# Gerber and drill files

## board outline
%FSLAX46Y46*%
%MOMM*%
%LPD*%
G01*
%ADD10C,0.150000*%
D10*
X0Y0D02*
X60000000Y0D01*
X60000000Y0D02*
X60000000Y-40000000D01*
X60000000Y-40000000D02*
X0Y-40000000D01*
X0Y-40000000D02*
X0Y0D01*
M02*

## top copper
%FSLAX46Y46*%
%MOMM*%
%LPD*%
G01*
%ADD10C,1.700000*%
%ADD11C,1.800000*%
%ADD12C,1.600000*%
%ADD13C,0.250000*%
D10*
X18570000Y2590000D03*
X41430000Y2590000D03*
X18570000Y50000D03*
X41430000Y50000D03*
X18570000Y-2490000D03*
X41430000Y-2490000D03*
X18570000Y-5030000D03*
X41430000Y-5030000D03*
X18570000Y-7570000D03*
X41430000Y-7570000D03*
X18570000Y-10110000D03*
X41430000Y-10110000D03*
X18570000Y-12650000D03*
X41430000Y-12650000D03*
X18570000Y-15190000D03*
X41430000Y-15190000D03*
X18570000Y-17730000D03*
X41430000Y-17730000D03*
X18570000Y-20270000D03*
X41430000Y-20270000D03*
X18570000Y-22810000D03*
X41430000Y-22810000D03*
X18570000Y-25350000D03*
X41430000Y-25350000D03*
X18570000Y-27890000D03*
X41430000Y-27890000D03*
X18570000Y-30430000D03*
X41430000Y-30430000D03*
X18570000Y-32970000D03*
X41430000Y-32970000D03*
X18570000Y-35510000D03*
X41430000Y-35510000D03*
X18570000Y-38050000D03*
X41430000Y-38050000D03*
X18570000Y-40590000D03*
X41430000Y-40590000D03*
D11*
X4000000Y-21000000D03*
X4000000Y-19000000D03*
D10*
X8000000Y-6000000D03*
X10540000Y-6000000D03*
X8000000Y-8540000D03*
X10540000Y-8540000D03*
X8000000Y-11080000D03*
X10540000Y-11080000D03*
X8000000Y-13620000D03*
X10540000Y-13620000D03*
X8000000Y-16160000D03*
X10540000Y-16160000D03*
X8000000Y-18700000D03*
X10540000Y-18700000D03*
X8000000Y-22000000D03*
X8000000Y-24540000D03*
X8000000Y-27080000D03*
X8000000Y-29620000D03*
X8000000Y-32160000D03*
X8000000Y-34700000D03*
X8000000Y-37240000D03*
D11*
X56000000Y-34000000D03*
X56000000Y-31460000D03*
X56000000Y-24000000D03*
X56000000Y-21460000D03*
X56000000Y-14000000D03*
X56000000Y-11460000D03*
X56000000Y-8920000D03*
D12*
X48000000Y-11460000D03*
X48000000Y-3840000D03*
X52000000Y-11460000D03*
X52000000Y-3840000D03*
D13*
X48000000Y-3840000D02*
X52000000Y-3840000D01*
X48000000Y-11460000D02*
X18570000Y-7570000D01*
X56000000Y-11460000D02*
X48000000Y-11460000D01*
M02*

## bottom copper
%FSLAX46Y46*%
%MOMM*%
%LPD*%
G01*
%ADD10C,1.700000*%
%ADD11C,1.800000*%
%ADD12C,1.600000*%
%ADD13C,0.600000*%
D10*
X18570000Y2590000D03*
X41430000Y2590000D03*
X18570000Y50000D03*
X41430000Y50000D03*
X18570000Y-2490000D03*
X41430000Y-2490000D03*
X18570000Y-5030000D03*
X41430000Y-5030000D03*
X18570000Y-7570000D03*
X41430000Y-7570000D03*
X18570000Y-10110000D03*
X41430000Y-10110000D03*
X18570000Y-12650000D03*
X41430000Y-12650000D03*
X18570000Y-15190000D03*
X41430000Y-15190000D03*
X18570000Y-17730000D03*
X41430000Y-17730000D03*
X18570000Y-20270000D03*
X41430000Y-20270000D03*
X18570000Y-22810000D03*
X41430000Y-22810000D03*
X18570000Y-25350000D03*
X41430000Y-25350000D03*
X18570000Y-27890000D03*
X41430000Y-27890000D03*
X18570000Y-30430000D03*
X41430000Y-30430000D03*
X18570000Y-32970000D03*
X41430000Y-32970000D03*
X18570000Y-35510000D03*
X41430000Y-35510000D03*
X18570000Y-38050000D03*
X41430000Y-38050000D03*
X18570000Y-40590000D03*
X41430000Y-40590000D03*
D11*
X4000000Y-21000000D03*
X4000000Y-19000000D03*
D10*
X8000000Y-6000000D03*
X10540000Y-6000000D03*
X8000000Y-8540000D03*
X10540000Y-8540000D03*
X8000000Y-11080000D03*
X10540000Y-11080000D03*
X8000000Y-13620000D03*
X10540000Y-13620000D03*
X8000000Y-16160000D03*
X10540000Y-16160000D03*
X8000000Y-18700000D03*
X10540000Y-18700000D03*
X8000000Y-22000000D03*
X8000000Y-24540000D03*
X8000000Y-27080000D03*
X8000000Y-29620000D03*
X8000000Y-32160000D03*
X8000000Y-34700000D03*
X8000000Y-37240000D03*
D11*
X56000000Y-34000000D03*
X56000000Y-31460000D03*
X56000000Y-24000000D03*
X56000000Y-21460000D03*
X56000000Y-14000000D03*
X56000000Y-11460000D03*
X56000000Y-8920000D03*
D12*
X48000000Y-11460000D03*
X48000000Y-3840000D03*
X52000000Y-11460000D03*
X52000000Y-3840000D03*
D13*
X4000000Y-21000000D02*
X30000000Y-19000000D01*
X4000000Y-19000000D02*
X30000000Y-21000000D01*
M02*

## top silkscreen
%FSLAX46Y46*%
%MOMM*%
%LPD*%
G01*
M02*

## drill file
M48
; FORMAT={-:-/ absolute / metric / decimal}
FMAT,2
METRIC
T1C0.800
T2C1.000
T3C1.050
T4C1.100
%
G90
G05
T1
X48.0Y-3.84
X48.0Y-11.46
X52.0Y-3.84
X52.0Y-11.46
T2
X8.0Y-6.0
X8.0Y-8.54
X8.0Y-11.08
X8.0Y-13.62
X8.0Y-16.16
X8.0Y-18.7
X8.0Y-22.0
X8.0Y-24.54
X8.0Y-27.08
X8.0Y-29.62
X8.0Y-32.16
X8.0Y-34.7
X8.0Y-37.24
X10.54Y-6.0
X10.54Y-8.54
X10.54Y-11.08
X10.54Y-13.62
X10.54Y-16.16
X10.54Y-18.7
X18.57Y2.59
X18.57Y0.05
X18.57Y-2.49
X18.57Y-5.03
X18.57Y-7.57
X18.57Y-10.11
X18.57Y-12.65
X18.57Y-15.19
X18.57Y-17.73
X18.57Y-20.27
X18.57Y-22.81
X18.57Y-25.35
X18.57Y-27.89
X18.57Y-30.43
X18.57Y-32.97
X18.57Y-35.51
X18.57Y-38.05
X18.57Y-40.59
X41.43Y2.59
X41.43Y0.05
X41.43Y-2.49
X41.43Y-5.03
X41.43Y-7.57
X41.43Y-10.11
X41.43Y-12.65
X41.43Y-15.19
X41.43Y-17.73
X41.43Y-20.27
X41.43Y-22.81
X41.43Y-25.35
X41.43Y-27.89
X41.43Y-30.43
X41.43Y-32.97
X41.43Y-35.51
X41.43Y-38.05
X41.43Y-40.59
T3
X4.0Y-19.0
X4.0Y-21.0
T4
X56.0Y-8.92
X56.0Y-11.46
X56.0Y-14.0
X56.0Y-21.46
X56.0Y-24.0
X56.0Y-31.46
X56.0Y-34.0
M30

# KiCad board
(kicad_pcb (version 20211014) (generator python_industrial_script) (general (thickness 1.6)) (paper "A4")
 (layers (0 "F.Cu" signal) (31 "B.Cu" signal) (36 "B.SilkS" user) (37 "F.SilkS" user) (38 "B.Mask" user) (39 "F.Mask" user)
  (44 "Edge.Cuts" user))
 (gr_line (start 0 0) (end 60.0 0) (layer "Edge.Cuts") (width 0.15))
 (gr_line (start 60.0 0) (end 60.0 40.0) (layer "Edge.Cuts") (width 0.15))
 (gr_line (start 60.0 40.0) (end 0 40.0) (layer "Edge.Cuts") (width 0.15))
 (gr_line (start 0 40.0) (end 0 0) (layer "Edge.Cuts") (width 0.15))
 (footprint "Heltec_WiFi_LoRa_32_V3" (layer "F.Cu") (at 0 0)
  (pad "1" thru_hole circle (at 18.5700 -2.5900) (size 1.7 1.7) (drill 1.0) (layers *.Cu *.Mask))
  (pad "19" thru_hole circle (at 41.4300 -2.5900) (size 1.7 1.7) (drill 1.0) (layers *.Cu *.Mask))
  (pad "2" thru_hole circle (at 18.5700 -0.0500) (size 1.7 1.7) (drill 1.0) (layers *.Cu *.Mask))
  (pad "20" thru_hole circle (at 41.4300 -0.0500) (size 1.7 1.7) (drill 1.0) (layers *.Cu *.Mask))
  (pad "3" thru_hole circle (at 18.5700 2.4900) (size 1.7 1.7) (drill 1.0) (layers *.Cu *.Mask))
  (pad "21" thru_hole circle (at 41.4300 2.4900) (size 1.7 1.7) (drill 1.0) (layers *.Cu *.Mask))
  (pad "4" thru_hole circle (at 18.5700 5.0300) (size 1.7 1.7) (drill 1.0) (layers *.Cu *.Mask))
  (pad "22" thru_hole circle (at 41.4300 5.0300) (size 1.7 1.7) (drill 1.0) (layers *.Cu *.Mask))
  (pad "5" thru_hole circle (at 18.5700 7.5700) (size 1.7 1.7) (drill 1.0) (layers *.Cu *.Mask))
  (pad "23" thru_hole circle (at 41.4300 7.5700) (size 1.7 1.7) (drill 1.0) (layers *.Cu *.Mask))
  (pad "6" thru_hole circle (at 18.5700 10.1100) (size 1.7 1.7) (drill 1.0) (layers *.Cu *.Mask))
  (pad "24" thru_hole circle (at 41.4300 10.1100) (size 1.7 1.7) (drill 1.0) (layers *.Cu *.Mask))
  (pad "7" thru_hole circle (at 18.5700 12.6500) (size 1.7 1.7) (drill 1.0) (layers *.Cu *.Mask))
  (pad "25" thru_hole circle (at 41.4300 12.6500) (size 1.7 1.7) (drill 1.0) (layers *.Cu *.Mask))
  (pad "8" thru_hole circle (at 18.5700 15.1900) (size 1.7 1.7) (drill 1.0) (layers *.Cu *.Mask))
  (pad "26" thru_hole circle (at 41.4300 15.1900) (size 1.7 1.7) (drill 1.0) (layers *.Cu *.Mask))
  (pad "9" thru_hole circle (at 18.5700 17.7300) (size 1.7 1.7) (drill 1.0) (layers *.Cu *.Mask))
  (pad "27" thru_hole circle (at 41.4300 17.7300) (size 1.7 1.7) (drill 1.0) (layers *.Cu *.Mask))
  (pad "10" thru_hole circle (at 18.5700 20.2700) (size 1.7 1.7) (drill 1.0) (layers *.Cu *.Mask))
  (pad "28" thru_hole circle (at 41.4300 20.2700) (size 1.7 1.7) (drill 1.0) (layers *.Cu *.Mask))
  (pad "11" thru_hole circle (at 18.5700 22.8100) (size 1.7 1.7) (drill 1.0) (layers *.Cu *.Mask))
  (pad "29" thru_hole circle (at 41.4300 22.8100) (size 1.7 1.7) (drill 1.0) (layers *.Cu *.Mask))
  (pad "12" thru_hole circle (at 18.5700 25.3500) (size 1.7 1.7) (drill 1.0) (layers *.Cu *.Mask))
  (pad "30" thru_hole circle (at 41.4300 25.3500) (size 1.7 1.7) (drill 1.0) (layers *.Cu *.Mask))
  (pad "13" thru_hole circle (at 18.5700 27.8900) (size 1.7 1.7) (drill 1.0) (layers *.Cu *.Mask))
  (pad "31" thru_hole circle (at 41.4300 27.8900) (size 1.7 1.7) (drill 1.0) (layers *.Cu *.Mask))
  (pad "14" thru_hole circle (at 18.5700 30.4300) (size 1.7 1.7) (drill 1.0) (layers *.Cu *.Mask))
  (pad "32" thru_hole circle (at 41.4300 30.4300) (size 1.7 1.7) (drill 1.0) (layers *.Cu *.Mask))
  (pad "15" thru_hole circle (at 18.5700 32.9700) (size 1.7 1.7) (drill 1.0) (layers *.Cu *.Mask))
  (pad "33" thru_hole circle (at 41.4300 32.9700) (size 1.7 1.7) (drill 1.0) (layers *.Cu *.Mask))
  (pad "16" thru_hole circle (at 18.5700 35.5100) (size 1.7 1.7) (drill 1.0) (layers *.Cu *.Mask))
  (pad "34" thru_hole circle (at 41.4300 35.5100) (size 1.7 1.7) (drill 1.0) (layers *.Cu *.Mask))
  (pad "17" thru_hole circle (at 18.5700 38.0500) (size 1.7 1.7) (drill 1.0) (layers *.Cu *.Mask))
  (pad "35" thru_hole circle (at 41.4300 38.0500) (size 1.7 1.7) (drill 1.0) (layers *.Cu *.Mask))
  (pad "18" thru_hole circle (at 18.5700 40.5900) (size 1.7 1.7) (drill 1.0) (layers *.Cu *.Mask))
  (pad "36" thru_hole circle (at 41.4300 40.5900) (size 1.7 1.7) (drill 1.0) (layers *.Cu *.Mask)))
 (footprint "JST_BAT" (layer "F.Cu") (at 0 0)
  (pad "1" thru_hole circle (at 4.00 21.00) (size 1.8 1.8) (drill 1.05) (layers *.Cu *.Mask))
  (pad "2" thru_hole circle (at 4.00 19.00) (size 1.8 1.8) (drill 1.05) (layers *.Cu *.Mask)))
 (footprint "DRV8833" (layer "F.Cu") (at 0 0)
  (pad "1" thru_hole circle (at 8.00 6.00) (size 1.7 1.7) (drill 1.0) (layers *.Cu *.Mask))
  (pad "7" thru_hole circle (at 10.54 6.00) (size 1.7 1.7) (drill 1.0) (layers *.Cu *.Mask))
  (pad "2" thru_hole circle (at 8.00 8.54) (size 1.7 1.7) (drill 1.0) (layers *.Cu *.Mask))
  (pad "8" thru_hole circle (at 10.54 8.54) (size 1.7 1.7) (drill 1.0) (layers *.Cu *.Mask))
  (pad "3" thru_hole circle (at 8.00 11.08) (size 1.7 1.7) (drill 1.0) (layers *.Cu *.Mask))
  (pad "9" thru_hole circle (at 10.54 11.08) (size 1.7 1.7) (drill 1.0) (layers *.Cu *.Mask))
  (pad "4" thru_hole circle (at 8.00 13.62) (size 1.7 1.7) (drill 1.0) (layers *.Cu *.Mask))
  (pad "10" thru_hole circle (at 10.54 13.62) (size 1.7 1.7) (drill 1.0) (layers *.Cu *.Mask))
  (pad "5" thru_hole circle (at 8.00 16.16) (size 1.7 1.7) (drill 1.0) (layers *.Cu *.Mask))
  (pad "11" thru_hole circle (at 10.54 16.16) (size 1.7 1.7) (drill 1.0) (layers *.Cu *.Mask))
  (pad "6" thru_hole circle (at 8.00 18.70) (size 1.7 1.7) (drill 1.0) (layers *.Cu *.Mask))
  (pad "12" thru_hole circle (at 10.54 18.70) (size 1.7 1.7) (drill 1.0) (layers *.Cu *.Mask)))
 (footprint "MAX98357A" (layer "F.Cu") (at 0 0)
  (pad "1" thru_hole circle (at 8.00 22.00) (size 1.7 1.7) (drill 1.0) (layers *.Cu *.Mask))
  (pad "2" thru_hole circle (at 8.00 24.54) (size 1.7 1.7) (drill 1.0) (layers *.Cu *.Mask))
  (pad "3" thru_hole circle (at 8.00 27.08) (size 1.7 1.7) (drill 1.0) (layers *.Cu *.Mask))
  (pad "4" thru_hole circle (at 8.00 29.62) (size 1.7 1.7) (drill 1.0) (layers *.Cu *.Mask))
  (pad "5" thru_hole circle (at 8.00 32.16) (size 1.7 1.7) (drill 1.0) (layers *.Cu *.Mask))
  (pad "6" thru_hole circle (at 8.00 34.70) (size 1.7 1.7) (drill 1.0) (layers *.Cu *.Mask))
  (pad "7" thru_hole circle (at 8.00 37.24) (size 1.7 1.7) (drill 1.0) (layers *.Cu *.Mask)))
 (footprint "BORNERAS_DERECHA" (layer "F.Cu") (at 0 0)
  (pad "SOL_1" thru_hole circle (at 56.00 34.00) (size 1.8 1.8) (drill 1.1) (layers *.Cu *.Mask))
  (pad "SOL_2" thru_hole circle (at 56.00 31.46) (size 1.8 1.8) (drill 1.1) (layers *.Cu *.Mask))
  (pad "SPK_1" thru_hole circle (at 56.00 24.00) (size 1.8 1.8) (drill 1.1) (layers *.Cu *.Mask))
  (pad "SPK_2" thru_hole circle (at 56.00 21.46) (size 1.8 1.8) (drill 1.1) (layers *.Cu *.Mask))
  (pad "FLOW_VCC" thru_hole circle (at 56.00 14.00) (size 1.8 1.8) (drill 1.1) (layers *.Cu *.Mask))
  (pad "FLOW_SIG" thru_hole circle (at 56.00 11.46) (size 1.8 1.8) (drill 1.1) (layers *.Cu *.Mask))
  (pad "FLOW_GND" thru_hole circle (at 56.00 8.92) (size 1.8 1.8) (drill 1.1) (layers *.Cu *.Mask)))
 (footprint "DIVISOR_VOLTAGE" (layer "F.Cu") (at 0 0)
  (pad "R1_1" thru_hole circle (at 48.00 11.46) (size 1.6 1.6) (drill 0.8) (layers *.Cu *.Mask))
  (pad "R1_2" thru_hole circle (at 48.00 3.84) (size 1.6 1.6) (drill 0.8) (layers *.Cu *.Mask))
  (pad "R2_1" thru_hole circle (at 52.00 11.46) (size 1.6 1.6) (drill 0.8) (layers *.Cu *.Mask))
  (pad "R2_2" thru_hole circle (at 52.00 3.84) (size 1.6 1.6) (drill 0.8) (layers *.Cu *.Mask)))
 (segment (start 48.00 3.84) (end 52.00 3.84) (width 0.25) (layer "F.Cu") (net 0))
 (segment (start 48.00 11.46) (end 18.5700 7.5700) (width 0.25) (layer "F.Cu") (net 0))
 (segment (start 56.00 11.46) (end 48.00 11.46) (width 0.25) (layer "F.Cu") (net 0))
 (segment (start 4.00 21.00) (end 30.00 19.00) (width 0.60) (layer "B.Cu") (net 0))
 (segment (start 4.00 19.00) (end 30.00 21.00) (width 0.60) (layer "B.Cu") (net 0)))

